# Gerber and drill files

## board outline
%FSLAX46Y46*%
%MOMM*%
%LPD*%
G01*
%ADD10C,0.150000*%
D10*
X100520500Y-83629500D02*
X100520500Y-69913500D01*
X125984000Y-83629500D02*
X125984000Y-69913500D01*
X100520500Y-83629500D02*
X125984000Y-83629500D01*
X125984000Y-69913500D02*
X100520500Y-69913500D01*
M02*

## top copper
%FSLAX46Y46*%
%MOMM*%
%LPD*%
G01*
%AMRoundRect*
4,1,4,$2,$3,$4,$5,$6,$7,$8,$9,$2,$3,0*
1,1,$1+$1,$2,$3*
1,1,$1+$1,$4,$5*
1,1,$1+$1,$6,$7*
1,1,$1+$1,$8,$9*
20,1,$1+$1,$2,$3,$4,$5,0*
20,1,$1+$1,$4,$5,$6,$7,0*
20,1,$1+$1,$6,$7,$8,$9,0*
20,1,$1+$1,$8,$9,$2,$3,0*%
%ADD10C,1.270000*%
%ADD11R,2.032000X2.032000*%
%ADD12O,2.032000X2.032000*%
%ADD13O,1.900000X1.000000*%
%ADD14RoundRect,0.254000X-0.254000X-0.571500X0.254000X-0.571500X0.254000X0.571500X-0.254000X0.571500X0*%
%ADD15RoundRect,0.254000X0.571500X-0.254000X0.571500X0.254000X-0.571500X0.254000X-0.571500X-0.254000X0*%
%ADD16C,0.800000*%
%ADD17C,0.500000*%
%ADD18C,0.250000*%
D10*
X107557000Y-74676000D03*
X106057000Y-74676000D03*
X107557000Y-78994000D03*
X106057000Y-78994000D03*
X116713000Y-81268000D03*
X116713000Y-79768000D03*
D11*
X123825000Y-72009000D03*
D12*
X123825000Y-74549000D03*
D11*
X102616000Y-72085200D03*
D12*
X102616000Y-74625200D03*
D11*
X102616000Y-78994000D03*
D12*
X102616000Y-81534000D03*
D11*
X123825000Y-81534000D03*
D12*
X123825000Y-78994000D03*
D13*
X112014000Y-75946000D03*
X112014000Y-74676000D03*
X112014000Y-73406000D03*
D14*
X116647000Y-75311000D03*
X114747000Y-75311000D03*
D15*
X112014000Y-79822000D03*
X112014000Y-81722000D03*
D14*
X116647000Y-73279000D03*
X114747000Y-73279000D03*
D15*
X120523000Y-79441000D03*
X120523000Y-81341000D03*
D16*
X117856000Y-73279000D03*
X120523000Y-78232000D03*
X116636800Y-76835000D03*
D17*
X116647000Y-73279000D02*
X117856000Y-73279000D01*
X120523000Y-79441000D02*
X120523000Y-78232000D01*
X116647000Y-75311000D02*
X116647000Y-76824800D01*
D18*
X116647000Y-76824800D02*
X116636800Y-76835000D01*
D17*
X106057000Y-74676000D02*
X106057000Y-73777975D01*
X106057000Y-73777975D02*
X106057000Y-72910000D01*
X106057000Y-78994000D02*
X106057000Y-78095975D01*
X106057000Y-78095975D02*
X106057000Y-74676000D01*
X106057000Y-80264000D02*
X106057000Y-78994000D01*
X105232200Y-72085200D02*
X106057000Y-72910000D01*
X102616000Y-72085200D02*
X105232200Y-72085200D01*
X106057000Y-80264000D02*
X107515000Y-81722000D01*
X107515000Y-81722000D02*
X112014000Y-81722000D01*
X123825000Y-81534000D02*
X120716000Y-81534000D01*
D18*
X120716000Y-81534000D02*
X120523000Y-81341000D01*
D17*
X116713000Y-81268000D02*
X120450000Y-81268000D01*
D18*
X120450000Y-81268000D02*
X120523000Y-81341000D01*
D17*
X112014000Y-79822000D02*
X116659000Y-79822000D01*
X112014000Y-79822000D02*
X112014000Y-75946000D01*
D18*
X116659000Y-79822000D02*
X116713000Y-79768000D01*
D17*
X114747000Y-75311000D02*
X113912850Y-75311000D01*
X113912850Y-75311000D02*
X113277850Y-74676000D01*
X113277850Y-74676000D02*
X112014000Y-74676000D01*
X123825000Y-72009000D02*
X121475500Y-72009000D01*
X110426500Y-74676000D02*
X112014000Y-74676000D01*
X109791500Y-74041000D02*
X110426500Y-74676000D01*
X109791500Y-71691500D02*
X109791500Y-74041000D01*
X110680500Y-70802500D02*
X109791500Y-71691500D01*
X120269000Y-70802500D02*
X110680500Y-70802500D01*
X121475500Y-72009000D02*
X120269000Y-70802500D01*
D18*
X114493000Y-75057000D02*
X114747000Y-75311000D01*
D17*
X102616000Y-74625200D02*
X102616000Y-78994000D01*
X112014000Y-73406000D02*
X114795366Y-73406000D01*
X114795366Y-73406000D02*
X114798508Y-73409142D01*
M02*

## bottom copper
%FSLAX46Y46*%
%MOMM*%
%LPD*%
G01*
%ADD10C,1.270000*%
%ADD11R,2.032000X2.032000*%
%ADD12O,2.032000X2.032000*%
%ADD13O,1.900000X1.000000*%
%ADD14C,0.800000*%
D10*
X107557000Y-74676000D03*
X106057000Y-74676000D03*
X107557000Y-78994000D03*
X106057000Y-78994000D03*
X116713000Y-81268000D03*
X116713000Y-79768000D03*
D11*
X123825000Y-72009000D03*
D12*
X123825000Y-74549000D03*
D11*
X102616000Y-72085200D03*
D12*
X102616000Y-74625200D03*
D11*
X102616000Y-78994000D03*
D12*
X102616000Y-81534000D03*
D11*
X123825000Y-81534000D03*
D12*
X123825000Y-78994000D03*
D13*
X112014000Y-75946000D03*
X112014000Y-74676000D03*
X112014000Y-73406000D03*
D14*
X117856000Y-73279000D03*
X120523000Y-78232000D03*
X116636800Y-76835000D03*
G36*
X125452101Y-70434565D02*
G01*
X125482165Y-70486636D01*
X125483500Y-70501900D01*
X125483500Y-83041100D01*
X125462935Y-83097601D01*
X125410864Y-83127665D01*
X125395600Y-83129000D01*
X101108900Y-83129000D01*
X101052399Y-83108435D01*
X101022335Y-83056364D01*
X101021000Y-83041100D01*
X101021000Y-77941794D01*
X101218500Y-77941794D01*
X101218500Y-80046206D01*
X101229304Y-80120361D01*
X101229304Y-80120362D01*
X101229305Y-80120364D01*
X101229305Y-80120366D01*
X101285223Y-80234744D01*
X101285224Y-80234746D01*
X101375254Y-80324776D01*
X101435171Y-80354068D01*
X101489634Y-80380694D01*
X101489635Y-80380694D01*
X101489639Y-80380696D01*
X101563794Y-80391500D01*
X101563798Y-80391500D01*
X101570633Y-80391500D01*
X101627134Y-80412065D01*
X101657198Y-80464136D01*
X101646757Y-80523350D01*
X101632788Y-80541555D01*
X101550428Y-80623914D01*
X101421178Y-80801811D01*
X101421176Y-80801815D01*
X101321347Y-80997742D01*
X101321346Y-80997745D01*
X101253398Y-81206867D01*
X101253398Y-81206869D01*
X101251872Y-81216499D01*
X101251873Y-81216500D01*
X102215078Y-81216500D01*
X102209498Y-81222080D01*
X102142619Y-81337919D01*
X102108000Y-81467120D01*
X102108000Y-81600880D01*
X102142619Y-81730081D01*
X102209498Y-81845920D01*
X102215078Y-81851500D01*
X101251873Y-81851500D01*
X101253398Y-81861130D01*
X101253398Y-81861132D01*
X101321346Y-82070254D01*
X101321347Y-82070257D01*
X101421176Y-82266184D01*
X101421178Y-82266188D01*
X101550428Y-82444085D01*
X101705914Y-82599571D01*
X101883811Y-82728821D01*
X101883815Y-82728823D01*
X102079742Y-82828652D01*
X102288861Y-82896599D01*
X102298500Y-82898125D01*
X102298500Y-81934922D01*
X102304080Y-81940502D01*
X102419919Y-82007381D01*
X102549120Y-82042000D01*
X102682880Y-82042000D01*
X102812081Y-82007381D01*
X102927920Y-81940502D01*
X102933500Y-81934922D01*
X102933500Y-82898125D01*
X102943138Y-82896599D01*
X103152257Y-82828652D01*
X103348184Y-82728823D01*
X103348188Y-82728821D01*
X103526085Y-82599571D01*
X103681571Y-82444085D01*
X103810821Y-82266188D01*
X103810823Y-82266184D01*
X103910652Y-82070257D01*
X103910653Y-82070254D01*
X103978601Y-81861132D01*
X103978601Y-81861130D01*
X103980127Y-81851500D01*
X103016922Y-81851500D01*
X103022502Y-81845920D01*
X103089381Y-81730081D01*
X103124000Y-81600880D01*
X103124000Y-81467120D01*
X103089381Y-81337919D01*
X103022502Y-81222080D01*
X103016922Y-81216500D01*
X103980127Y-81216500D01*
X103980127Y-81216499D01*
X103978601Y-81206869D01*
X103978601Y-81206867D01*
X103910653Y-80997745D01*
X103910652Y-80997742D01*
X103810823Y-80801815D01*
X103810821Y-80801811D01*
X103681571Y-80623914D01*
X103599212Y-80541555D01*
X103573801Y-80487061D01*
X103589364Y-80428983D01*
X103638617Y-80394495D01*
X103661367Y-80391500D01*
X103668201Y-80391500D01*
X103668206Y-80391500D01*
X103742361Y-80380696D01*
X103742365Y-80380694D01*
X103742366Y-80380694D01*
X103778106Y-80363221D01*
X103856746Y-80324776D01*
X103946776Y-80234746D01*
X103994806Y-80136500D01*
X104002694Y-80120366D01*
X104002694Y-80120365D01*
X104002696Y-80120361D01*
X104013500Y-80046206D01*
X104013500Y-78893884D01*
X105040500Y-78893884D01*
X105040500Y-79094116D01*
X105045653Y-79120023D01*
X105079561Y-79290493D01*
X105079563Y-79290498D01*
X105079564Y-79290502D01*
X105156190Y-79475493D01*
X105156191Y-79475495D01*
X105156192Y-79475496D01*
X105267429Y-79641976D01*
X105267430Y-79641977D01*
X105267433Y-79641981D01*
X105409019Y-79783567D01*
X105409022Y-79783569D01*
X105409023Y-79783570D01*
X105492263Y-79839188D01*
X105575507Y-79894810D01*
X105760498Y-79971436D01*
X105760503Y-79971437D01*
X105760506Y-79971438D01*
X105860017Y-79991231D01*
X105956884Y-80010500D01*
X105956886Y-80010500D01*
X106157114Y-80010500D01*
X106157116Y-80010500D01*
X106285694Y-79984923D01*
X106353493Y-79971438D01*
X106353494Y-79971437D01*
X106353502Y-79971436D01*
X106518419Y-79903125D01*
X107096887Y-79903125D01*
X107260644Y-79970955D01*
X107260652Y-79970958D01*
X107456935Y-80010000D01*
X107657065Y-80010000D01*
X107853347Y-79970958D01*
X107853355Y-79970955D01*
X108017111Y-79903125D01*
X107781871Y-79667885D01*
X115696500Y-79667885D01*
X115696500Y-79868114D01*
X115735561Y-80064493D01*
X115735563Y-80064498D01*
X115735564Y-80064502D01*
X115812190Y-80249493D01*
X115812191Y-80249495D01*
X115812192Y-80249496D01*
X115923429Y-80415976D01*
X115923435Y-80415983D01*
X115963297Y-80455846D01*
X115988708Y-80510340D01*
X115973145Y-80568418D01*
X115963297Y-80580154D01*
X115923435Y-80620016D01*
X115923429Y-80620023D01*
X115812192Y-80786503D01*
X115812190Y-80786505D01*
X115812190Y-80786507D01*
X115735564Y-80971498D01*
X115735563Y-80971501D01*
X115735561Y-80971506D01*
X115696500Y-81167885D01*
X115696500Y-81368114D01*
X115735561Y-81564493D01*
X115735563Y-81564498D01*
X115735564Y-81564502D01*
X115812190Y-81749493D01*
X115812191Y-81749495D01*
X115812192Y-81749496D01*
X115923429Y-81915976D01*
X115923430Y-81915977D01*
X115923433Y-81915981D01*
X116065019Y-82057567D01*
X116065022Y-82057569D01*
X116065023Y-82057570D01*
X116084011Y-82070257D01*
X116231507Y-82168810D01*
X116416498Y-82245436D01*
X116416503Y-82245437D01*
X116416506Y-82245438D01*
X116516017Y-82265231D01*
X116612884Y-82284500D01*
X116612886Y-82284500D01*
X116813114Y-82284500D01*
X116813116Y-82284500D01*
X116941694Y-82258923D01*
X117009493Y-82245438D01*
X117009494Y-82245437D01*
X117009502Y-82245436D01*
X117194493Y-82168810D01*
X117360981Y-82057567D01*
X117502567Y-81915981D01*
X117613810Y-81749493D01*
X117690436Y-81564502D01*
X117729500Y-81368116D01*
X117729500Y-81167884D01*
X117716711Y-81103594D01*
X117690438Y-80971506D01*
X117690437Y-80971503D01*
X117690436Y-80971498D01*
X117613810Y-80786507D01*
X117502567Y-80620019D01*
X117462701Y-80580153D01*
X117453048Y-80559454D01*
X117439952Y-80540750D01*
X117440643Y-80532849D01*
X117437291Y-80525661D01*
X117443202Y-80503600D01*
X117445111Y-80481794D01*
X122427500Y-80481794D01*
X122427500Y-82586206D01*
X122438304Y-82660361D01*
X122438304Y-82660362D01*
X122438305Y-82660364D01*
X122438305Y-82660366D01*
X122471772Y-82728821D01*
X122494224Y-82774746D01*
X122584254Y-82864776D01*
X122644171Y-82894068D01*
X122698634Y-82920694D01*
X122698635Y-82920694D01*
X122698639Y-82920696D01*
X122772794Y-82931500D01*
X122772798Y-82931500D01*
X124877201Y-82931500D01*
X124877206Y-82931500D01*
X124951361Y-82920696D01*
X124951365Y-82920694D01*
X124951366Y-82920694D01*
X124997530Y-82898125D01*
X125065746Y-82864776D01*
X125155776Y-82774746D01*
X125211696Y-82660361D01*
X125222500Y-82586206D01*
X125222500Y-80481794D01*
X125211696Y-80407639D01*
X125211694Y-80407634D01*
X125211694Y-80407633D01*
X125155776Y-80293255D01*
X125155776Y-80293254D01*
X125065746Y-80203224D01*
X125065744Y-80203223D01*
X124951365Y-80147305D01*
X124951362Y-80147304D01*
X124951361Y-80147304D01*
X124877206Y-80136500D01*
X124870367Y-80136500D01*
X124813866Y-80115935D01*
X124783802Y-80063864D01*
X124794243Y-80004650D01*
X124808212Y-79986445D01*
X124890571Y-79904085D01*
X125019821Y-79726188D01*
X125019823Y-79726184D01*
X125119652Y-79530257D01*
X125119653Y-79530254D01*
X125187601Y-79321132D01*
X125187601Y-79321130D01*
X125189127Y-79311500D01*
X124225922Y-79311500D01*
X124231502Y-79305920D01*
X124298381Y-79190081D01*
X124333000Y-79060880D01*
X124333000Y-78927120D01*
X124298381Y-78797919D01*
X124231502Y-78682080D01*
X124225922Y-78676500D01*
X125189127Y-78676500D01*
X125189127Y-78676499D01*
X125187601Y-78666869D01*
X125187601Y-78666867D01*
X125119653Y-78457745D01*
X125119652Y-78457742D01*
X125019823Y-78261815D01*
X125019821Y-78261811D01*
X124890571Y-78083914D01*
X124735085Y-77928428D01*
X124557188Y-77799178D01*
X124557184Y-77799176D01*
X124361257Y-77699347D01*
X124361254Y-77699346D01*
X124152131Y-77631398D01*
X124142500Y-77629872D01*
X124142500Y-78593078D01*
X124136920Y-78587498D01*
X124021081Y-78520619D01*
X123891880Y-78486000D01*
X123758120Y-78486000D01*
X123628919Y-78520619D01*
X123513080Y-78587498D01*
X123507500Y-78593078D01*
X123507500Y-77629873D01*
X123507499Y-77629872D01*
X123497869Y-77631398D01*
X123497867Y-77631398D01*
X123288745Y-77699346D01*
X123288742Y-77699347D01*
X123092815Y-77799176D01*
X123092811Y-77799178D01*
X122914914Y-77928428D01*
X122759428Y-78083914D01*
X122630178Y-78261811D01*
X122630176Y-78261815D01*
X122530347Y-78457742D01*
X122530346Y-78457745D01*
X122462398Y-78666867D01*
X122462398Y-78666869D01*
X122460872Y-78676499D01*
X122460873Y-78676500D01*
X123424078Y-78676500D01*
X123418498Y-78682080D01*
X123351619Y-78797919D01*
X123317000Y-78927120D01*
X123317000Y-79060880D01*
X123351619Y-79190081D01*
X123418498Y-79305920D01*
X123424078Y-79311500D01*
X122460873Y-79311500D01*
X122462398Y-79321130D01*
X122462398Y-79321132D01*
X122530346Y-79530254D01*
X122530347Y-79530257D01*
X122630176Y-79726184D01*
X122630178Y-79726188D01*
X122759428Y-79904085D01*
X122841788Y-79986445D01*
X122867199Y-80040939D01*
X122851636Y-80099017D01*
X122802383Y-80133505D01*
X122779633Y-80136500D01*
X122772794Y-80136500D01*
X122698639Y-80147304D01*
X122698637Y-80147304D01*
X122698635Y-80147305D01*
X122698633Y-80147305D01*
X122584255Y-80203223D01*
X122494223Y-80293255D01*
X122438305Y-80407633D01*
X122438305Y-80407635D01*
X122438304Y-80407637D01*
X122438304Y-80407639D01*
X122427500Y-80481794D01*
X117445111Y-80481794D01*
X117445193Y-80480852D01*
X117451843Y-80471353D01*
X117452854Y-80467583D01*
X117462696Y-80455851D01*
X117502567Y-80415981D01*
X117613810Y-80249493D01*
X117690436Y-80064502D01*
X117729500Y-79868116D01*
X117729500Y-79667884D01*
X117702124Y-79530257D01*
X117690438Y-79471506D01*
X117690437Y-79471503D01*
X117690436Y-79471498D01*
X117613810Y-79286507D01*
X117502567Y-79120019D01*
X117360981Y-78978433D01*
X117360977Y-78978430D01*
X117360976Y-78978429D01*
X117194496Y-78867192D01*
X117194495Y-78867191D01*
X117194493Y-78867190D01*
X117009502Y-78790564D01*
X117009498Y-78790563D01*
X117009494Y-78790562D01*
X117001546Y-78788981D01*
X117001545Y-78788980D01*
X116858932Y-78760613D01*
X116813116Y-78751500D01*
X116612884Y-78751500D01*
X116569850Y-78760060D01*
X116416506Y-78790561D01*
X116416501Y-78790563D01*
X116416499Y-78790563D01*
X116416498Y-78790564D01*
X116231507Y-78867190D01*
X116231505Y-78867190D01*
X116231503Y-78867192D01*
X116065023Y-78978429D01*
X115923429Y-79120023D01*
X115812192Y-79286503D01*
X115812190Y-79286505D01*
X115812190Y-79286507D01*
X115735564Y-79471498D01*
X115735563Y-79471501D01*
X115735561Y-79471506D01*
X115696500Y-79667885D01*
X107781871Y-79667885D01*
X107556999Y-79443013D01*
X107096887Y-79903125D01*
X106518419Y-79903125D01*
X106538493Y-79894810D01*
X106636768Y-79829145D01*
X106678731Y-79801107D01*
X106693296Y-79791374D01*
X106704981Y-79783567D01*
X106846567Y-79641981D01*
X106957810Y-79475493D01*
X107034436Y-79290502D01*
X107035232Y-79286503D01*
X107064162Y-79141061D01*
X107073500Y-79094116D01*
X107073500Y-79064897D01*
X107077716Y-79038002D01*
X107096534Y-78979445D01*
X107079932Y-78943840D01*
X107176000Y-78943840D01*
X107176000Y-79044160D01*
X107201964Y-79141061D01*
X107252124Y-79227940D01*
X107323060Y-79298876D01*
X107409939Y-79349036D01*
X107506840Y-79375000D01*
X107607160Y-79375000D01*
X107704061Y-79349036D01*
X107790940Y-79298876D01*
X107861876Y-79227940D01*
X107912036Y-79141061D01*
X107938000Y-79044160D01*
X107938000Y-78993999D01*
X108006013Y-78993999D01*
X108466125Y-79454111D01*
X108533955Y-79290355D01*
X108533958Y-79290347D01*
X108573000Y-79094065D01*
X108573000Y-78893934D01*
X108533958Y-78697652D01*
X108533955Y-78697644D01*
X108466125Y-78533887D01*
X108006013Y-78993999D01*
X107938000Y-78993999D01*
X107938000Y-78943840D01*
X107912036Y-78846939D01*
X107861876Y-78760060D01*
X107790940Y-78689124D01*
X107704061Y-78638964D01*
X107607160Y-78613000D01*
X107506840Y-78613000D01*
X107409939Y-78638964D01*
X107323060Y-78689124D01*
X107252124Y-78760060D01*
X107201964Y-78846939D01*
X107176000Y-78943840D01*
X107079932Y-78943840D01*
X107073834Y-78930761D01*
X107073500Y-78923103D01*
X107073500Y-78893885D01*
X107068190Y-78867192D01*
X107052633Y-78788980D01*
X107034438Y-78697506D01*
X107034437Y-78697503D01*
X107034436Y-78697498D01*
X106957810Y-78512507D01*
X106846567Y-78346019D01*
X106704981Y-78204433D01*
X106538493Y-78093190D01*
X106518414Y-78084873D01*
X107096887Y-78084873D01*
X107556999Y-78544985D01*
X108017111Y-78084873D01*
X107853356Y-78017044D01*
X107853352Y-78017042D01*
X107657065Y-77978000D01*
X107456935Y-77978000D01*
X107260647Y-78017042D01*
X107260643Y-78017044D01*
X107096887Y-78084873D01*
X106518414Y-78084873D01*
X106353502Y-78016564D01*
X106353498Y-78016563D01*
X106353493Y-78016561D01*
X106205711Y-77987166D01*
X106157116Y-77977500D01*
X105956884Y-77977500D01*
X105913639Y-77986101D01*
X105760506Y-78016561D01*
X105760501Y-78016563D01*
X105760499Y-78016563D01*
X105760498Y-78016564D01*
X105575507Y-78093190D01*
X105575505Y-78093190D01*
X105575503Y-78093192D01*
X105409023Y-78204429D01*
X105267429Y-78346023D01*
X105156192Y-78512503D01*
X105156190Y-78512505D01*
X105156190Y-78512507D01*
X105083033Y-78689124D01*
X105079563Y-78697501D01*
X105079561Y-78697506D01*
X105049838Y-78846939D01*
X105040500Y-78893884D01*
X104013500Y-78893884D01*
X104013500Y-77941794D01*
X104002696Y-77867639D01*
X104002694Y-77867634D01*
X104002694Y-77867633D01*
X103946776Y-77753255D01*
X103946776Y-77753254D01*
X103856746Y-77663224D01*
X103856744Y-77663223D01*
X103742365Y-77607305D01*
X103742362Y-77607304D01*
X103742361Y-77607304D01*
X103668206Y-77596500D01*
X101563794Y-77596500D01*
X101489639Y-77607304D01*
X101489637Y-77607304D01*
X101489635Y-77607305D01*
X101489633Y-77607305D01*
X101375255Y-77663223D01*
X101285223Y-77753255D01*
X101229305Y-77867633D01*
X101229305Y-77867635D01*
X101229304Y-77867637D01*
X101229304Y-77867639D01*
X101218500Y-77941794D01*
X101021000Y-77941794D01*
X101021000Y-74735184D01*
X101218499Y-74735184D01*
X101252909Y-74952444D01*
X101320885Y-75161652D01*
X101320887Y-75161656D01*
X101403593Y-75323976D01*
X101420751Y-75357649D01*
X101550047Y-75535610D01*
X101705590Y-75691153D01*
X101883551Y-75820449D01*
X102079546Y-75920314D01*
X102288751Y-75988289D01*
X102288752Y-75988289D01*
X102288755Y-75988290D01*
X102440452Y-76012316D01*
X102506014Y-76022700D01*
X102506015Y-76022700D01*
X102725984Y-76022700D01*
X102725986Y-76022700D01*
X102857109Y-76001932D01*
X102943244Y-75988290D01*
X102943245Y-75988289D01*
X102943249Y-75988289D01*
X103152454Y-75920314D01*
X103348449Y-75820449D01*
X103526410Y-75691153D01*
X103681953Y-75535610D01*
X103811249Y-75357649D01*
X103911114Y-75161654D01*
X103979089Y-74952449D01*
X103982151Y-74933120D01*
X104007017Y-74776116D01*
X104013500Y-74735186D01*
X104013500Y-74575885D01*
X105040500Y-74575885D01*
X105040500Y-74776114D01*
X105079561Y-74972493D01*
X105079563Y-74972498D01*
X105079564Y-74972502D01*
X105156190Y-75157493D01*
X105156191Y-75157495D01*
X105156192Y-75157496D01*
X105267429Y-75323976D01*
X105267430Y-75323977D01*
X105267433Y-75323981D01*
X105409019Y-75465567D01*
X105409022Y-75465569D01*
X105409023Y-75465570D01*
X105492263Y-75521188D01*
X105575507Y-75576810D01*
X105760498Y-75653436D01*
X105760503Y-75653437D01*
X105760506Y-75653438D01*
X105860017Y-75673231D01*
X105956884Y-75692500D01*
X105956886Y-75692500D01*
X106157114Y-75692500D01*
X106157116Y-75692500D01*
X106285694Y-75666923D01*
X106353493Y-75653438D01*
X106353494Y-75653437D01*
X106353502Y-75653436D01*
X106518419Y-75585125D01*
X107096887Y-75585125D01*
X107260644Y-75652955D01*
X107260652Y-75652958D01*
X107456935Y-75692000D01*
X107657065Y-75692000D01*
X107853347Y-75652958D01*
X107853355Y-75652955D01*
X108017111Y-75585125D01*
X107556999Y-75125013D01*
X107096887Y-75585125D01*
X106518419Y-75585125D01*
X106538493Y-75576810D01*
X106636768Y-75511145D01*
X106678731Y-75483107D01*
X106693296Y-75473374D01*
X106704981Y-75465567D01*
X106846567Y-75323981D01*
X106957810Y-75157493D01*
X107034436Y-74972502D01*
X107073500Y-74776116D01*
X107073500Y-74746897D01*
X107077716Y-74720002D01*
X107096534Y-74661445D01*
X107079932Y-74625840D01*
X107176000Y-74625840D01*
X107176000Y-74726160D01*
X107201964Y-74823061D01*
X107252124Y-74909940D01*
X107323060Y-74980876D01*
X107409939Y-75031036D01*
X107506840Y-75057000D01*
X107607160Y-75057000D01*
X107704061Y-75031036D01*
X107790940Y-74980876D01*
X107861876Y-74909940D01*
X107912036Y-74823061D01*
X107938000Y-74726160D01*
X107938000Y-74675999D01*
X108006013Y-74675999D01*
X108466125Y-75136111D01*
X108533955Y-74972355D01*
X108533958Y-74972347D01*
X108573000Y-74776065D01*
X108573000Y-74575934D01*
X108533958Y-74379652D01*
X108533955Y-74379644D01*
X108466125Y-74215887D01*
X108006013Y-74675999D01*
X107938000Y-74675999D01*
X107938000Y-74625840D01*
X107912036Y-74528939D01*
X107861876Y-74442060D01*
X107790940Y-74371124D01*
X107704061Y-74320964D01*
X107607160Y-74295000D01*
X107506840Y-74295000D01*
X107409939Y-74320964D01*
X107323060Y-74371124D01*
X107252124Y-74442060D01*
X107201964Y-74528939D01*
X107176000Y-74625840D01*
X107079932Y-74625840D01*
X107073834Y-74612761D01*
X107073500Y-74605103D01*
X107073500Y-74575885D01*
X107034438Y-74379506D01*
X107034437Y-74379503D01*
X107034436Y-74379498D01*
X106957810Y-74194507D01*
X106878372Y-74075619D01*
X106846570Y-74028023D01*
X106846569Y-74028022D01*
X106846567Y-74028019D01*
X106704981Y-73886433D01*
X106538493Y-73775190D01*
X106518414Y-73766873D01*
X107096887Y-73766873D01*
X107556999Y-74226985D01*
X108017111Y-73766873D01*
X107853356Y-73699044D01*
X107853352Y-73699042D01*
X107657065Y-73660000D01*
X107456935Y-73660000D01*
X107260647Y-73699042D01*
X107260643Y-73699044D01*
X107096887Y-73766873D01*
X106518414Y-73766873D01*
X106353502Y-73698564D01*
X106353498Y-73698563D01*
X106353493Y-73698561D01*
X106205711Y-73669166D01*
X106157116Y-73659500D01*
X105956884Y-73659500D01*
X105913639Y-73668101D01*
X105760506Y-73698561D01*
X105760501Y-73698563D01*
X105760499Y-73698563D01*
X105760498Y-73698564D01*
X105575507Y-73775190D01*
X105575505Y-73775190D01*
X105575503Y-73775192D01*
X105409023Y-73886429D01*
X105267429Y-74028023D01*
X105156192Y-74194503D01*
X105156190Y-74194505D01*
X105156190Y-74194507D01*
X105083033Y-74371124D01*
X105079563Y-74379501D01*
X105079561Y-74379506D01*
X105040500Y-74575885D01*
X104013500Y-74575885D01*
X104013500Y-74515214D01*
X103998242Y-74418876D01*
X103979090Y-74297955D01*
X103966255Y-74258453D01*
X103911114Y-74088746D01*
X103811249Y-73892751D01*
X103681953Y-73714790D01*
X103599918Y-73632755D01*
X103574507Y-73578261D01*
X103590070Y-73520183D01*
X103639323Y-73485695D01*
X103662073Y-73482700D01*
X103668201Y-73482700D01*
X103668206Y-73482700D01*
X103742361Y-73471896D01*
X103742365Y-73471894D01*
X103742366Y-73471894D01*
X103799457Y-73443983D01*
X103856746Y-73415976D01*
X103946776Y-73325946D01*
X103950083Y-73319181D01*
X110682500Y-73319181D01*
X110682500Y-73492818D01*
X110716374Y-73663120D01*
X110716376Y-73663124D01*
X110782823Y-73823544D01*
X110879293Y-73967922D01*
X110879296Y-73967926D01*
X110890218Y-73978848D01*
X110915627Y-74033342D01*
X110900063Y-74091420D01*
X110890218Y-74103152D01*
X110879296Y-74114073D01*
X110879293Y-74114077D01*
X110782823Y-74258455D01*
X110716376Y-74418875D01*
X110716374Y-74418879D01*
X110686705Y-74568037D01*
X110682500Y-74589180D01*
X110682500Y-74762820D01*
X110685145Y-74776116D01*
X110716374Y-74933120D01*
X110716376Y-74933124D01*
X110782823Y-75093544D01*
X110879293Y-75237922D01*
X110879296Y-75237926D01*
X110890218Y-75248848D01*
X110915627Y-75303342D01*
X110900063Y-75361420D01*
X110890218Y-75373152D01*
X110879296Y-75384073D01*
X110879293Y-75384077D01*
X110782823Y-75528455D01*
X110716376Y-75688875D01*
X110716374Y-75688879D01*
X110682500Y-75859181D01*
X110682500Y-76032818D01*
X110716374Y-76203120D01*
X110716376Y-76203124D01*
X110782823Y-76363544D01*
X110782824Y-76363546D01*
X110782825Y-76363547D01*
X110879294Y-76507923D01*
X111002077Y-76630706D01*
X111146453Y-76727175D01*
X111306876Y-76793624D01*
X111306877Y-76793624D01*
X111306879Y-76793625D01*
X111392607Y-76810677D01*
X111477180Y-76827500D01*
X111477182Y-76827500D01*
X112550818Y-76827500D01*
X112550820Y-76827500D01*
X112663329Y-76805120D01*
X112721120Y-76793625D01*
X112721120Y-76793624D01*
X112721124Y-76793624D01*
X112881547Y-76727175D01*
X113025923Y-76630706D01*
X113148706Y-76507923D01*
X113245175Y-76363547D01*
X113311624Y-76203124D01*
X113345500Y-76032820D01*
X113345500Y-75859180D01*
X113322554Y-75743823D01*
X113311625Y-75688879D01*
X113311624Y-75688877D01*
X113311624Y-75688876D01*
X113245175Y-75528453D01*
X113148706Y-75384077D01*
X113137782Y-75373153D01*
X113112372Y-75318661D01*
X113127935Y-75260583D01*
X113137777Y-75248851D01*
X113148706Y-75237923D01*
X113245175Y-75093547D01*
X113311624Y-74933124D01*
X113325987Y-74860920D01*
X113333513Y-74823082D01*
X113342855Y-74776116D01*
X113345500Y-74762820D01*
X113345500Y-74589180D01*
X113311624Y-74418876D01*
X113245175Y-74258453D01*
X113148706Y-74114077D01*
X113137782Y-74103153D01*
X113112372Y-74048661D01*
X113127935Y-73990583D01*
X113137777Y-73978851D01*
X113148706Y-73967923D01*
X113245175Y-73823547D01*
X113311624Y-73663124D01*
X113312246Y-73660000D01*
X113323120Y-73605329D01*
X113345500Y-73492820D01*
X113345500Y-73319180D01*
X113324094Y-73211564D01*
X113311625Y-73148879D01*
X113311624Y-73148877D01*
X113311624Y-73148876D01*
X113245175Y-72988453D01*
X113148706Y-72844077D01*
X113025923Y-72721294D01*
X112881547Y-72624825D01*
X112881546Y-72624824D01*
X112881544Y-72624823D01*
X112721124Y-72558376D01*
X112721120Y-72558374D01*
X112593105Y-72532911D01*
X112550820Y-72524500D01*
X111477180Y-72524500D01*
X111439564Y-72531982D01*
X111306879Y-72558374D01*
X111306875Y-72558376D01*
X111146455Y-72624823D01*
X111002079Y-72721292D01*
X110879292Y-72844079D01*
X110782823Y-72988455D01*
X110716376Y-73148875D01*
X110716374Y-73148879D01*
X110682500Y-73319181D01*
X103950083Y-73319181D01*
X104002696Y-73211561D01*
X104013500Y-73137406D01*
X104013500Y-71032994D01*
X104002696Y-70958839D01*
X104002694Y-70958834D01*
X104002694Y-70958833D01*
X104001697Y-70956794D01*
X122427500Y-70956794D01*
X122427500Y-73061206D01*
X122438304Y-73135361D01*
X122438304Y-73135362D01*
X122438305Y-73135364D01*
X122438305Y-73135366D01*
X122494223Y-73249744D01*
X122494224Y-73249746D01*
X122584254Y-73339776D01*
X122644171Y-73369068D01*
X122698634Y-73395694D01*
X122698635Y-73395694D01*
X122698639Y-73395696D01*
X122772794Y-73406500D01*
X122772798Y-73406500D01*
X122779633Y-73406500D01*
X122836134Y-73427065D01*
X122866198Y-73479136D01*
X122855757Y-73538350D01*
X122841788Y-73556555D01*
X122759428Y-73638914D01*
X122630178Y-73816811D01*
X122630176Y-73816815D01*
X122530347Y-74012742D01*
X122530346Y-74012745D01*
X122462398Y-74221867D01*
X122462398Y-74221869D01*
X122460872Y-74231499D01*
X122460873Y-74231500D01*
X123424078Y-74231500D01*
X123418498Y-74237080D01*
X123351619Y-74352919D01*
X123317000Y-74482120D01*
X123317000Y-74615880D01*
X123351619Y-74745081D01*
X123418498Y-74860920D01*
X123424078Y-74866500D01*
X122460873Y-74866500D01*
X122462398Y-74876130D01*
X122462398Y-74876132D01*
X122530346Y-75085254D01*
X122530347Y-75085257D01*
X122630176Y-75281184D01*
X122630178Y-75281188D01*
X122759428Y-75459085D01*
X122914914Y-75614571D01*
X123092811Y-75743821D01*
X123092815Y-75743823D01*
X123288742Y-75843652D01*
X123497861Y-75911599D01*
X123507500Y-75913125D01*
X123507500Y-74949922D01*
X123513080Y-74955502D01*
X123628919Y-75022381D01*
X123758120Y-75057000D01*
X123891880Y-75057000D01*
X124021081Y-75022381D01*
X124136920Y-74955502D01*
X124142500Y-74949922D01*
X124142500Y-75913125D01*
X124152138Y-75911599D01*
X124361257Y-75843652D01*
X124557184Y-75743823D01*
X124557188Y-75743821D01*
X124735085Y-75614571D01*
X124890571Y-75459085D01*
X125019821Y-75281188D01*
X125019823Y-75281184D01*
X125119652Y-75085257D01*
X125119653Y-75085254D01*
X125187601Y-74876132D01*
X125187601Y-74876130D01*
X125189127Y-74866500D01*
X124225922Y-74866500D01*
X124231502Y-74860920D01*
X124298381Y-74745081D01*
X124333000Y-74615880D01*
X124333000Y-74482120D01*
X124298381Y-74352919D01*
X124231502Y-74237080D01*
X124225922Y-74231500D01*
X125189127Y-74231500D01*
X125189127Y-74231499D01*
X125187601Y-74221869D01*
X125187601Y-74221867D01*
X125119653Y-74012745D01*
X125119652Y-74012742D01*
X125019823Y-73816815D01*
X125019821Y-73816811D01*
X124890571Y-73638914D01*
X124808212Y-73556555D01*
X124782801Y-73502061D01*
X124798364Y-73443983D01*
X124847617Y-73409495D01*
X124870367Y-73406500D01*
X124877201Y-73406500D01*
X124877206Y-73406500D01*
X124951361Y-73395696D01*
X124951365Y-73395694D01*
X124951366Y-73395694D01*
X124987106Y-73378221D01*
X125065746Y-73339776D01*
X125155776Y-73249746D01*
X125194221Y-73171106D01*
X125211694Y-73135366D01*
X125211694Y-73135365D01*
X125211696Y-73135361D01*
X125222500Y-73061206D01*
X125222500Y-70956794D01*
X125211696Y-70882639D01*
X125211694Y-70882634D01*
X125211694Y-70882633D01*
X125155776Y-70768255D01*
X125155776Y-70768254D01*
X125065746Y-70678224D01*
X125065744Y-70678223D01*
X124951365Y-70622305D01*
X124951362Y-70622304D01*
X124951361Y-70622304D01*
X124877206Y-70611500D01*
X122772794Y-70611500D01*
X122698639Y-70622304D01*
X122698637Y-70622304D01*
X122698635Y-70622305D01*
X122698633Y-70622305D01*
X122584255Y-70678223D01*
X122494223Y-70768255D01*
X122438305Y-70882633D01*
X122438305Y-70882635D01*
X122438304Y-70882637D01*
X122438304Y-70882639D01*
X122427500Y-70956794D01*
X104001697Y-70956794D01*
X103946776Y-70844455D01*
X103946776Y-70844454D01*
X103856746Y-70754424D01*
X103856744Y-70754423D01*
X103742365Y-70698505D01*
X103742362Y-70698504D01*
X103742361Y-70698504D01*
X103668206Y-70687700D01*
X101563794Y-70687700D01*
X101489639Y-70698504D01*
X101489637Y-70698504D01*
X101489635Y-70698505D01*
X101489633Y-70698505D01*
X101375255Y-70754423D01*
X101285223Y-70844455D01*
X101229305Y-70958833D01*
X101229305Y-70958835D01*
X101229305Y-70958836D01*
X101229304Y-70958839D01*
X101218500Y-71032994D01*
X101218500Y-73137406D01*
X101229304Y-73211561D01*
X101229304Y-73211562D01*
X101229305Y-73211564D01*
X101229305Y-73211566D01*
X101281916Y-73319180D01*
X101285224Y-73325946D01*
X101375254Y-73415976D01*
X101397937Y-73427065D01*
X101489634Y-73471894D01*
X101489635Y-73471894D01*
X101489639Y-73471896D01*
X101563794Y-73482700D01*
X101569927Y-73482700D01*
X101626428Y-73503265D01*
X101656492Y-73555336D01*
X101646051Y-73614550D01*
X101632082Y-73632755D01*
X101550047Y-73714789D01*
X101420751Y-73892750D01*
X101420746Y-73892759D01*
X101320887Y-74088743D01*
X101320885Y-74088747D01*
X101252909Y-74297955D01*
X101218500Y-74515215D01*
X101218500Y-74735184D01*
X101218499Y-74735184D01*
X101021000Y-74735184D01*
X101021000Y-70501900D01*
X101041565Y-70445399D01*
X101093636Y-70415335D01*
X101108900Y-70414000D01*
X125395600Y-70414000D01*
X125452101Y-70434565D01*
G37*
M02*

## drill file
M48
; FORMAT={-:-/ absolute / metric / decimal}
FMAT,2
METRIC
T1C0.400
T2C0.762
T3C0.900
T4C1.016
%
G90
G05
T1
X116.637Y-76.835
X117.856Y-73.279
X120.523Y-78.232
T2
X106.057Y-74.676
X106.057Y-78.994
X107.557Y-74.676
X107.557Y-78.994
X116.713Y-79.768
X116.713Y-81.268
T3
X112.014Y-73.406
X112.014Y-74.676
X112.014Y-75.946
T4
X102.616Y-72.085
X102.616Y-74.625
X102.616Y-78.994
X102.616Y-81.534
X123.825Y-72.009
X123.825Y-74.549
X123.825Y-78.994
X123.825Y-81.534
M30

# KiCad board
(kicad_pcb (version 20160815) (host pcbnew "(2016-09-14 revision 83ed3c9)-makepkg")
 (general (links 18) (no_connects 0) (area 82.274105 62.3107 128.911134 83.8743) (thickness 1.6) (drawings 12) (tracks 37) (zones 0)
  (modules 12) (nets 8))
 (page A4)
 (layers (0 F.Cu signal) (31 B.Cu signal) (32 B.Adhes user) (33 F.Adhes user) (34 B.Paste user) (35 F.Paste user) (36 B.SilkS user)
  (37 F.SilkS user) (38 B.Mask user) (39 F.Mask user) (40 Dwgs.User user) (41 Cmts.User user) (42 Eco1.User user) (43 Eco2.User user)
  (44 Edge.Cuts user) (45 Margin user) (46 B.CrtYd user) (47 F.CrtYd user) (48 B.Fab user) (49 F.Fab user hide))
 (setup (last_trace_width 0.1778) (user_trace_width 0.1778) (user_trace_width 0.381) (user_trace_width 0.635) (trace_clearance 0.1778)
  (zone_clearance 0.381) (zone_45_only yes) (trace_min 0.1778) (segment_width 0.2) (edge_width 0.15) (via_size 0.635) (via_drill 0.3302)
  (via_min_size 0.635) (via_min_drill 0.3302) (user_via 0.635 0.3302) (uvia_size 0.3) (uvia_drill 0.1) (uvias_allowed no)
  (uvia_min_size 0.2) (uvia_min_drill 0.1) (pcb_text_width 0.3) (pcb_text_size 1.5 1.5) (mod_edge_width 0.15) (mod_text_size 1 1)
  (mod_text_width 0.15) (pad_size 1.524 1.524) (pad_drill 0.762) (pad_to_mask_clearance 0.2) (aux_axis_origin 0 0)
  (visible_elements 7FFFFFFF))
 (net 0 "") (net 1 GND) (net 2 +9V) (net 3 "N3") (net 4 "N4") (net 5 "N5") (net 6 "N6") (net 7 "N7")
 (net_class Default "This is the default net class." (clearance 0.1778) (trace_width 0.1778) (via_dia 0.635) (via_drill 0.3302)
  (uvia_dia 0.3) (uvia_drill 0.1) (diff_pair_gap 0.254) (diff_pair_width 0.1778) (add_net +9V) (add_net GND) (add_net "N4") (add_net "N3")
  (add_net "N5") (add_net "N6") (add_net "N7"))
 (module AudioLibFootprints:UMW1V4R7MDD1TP (layer F.Cu) (at 106.807 74.676)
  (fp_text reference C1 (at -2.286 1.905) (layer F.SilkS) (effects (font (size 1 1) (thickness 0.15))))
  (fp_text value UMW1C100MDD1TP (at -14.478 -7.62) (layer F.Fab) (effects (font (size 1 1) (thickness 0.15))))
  (pad 2 thru_hole circle (at 0.75 0) (size 1.27 1.27) (drill 0.762) (layers *.Cu *.Mask) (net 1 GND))
  (pad 1 thru_hole circle (at -0.75 0) (size 1.27 1.27) (drill 0.762) (layers *.Cu *.Mask) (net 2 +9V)))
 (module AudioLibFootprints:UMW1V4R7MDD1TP (layer F.Cu) (at 106.807 78.994)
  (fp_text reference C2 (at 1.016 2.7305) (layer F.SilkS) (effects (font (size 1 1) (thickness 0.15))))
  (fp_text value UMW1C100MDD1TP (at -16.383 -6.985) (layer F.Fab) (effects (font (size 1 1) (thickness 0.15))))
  (pad 2 thru_hole circle (at 0.75 0) (size 1.27 1.27) (drill 0.762) (layers *.Cu *.Mask) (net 1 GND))
  (pad 1 thru_hole circle (at -0.75 0) (size 1.27 1.27) (drill 0.762) (layers *.Cu *.Mask) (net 2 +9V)))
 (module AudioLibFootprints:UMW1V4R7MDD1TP (layer F.Cu) (at 116.713 80.518 270)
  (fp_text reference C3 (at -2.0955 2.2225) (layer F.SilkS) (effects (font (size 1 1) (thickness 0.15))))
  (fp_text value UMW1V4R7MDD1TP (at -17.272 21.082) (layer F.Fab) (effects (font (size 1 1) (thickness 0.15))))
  (pad 2 thru_hole circle (at 0.75 0 270) (size 1.27 1.27) (drill 0.762) (layers *.Cu *.Mask) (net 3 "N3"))
  (pad 1 thru_hole circle (at -0.75 0 270) (size 1.27 1.27) (drill 0.762) (layers *.Cu *.Mask) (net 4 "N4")))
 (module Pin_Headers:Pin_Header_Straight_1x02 (layer F.Cu) (at 123.825 72.009)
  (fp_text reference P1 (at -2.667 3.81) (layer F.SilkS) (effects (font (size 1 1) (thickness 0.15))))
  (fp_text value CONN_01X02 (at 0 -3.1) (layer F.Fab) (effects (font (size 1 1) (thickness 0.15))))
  (pad 1 thru_hole rect (at 0 0) (size 2.032 2.032) (drill 1.016) (layers *.Cu *.Mask F.SilkS) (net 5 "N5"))
  (pad 2 thru_hole oval (at 0 2.54) (size 2.032 2.032) (drill 1.016) (layers *.Cu *.Mask F.SilkS) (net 1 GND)))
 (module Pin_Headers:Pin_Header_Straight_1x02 (layer F.Cu) (at 102.616 72.0852)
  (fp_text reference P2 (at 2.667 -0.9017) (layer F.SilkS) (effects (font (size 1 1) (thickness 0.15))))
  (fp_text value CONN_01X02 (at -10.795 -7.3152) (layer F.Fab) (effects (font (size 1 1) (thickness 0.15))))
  (pad 1 thru_hole rect (at 0 0) (size 2.032 2.032) (drill 1.016) (layers *.Cu *.Mask F.SilkS) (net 2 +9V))
  (pad 2 thru_hole oval (at 0 2.54) (size 2.032 2.032) (drill 1.016) (layers *.Cu *.Mask F.SilkS) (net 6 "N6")))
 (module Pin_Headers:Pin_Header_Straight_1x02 (layer F.Cu) (at 102.616 78.994)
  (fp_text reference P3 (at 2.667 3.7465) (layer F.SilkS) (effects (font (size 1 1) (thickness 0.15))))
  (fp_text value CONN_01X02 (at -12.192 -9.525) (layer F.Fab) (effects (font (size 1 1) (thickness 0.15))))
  (pad 1 thru_hole rect (at 0 0) (size 2.032 2.032) (drill 1.016) (layers *.Cu *.Mask F.SilkS) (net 6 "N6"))
  (pad 2 thru_hole oval (at 0 2.54) (size 2.032 2.032) (drill 1.016) (layers *.Cu *.Mask F.SilkS) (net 1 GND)))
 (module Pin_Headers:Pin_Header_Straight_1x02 (layer F.Cu) (at 123.825 81.534 180)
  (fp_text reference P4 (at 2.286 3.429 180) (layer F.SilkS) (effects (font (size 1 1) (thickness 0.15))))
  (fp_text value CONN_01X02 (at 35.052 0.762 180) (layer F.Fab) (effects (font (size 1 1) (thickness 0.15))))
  (pad 1 thru_hole rect (at 0 0 180) (size 2.032 2.032) (drill 1.016) (layers *.Cu *.Mask F.SilkS) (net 3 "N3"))
  (pad 2 thru_hole oval (at 0 2.54 180) (size 2.032 2.032) (drill 1.016) (layers *.Cu *.Mask F.SilkS) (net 1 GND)))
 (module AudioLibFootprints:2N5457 (layer F.Cu) (at 112.014 74.676)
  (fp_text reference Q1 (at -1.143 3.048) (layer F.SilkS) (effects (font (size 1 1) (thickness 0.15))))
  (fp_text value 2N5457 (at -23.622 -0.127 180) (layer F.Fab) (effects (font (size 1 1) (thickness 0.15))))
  (pad 1 thru_hole oval (at 0 1.27) (size 1.9 1) (drill 0.9) (layers *.Cu *.Mask) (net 4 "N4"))
  (pad 2 thru_hole oval (at 0 0) (size 1.9 1) (drill 0.9) (layers *.Cu *.Mask) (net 5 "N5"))
  (pad 3 thru_hole oval (at 0 -1.27) (size 1.9 1) (drill 0.9) (layers *.Cu *.Mask) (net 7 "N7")))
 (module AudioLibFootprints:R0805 (layer F.Cu) (at 115.697 75.311)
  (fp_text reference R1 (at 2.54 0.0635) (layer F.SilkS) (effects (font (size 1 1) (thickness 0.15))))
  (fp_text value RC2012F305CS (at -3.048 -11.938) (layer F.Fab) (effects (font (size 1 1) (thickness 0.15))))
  (pad 2 smd roundrect (at 0.95 0) (size 1.016 1.651) (layers F.Cu F.Paste F.Mask) (roundrect_rratio 0.25) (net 1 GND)
   (solder_mask_margin 0.102))
  (pad 1 smd roundrect (at -0.95 0) (size 1.016 1.651) (layers F.Cu F.Paste F.Mask) (roundrect_rratio 0.25) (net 5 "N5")
   (solder_mask_margin 0.102)))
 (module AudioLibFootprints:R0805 (layer F.Cu) (at 112.014 80.772 90)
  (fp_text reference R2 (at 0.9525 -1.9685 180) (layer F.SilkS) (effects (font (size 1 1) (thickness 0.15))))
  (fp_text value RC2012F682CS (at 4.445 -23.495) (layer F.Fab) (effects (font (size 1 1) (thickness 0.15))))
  (pad 2 smd roundrect (at 0.95 0 90) (size 1.016 1.651) (layers F.Cu F.Paste F.Mask) (roundrect_rratio 0.25) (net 4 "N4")
   (solder_mask_margin 0.102))
  (pad 1 smd roundrect (at -0.95 0 90) (size 1.016 1.651) (layers F.Cu F.Paste F.Mask) (roundrect_rratio 0.25) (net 2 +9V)
   (solder_mask_margin 0.102)))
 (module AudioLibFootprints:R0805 (layer F.Cu) (at 115.697 73.279)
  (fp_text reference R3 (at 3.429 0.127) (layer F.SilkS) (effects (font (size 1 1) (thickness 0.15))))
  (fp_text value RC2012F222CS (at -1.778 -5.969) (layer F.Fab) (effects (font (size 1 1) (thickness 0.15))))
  (pad 2 smd roundrect (at 0.95 0) (size 1.016 1.651) (layers F.Cu F.Paste F.Mask) (roundrect_rratio 0.25) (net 1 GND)
   (solder_mask_margin 0.102))
  (pad 1 smd roundrect (at -0.95 0) (size 1.016 1.651) (layers F.Cu F.Paste F.Mask) (roundrect_rratio 0.25) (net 7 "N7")
   (solder_mask_margin 0.102)))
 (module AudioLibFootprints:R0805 (layer F.Cu) (at 120.523 80.391 90)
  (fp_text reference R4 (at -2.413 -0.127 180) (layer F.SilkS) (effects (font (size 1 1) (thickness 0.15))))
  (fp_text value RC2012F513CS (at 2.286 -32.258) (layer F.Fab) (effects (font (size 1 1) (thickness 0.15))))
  (pad 2 smd roundrect (at 0.95 0 90) (size 1.016 1.651) (layers F.Cu F.Paste F.Mask) (roundrect_rratio 0.25) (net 1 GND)
   (solder_mask_margin 0.102))
  (pad 1 smd roundrect (at -0.95 0 90) (size 1.016 1.651) (layers F.Cu F.Paste F.Mask) (roundrect_rratio 0.25) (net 3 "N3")
   (solder_mask_margin 0.102)))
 (gr_line (start 100.5205 83.6295) (end 100.5205 69.9135) (angle 90) (layer Edge.Cuts) (width 0.15))
 (gr_line (start 125.984 83.6295) (end 125.984 69.9135) (angle 90) (layer Edge.Cuts) (width 0.15))
 (gr_line (start 100.5205 83.6295) (end 125.984 83.6295) (angle 90) (layer Edge.Cuts) (width 0.15))
 (gr_line (start 125.984 69.9135) (end 100.5205 69.9135) (angle 90) (layer Edge.Cuts) (width 0.15))
 (segment (start 116.647 73.279) (end 117.856 73.279) (width 0.5) (layer F.Cu) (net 1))
 (via (at 117.856 73.279) (size 0.8) (drill 0.4) (layers F.Cu B.Cu) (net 1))
 (segment (start 120.523 79.441) (end 120.523 78.232) (width 0.5) (layer F.Cu) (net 1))
 (via (at 120.523 78.232) (size 0.8) (drill 0.4) (layers F.Cu B.Cu) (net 1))
 (segment (start 116.647 75.311) (end 116.647 76.8248) (width 0.5) (layer F.Cu) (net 1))
 (segment (start 116.647 76.8248) (end 116.6368 76.835) (width 0.25) (layer F.Cu) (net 1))
 (via (at 116.6368 76.835) (size 0.8) (drill 0.4) (layers F.Cu B.Cu) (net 1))
 (segment (start 106.057 74.676) (end 106.057 73.777975) (width 0.5) (layer F.Cu) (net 2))
 (segment (start 106.057 73.777975) (end 106.057 72.91) (width 0.5) (layer F.Cu) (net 2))
 (segment (start 106.057 78.994) (end 106.057 78.095975) (width 0.5) (layer F.Cu) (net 2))
 (segment (start 106.057 78.095975) (end 106.057 74.676) (width 0.5) (layer F.Cu) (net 2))
 (segment (start 106.057 80.264) (end 106.057 78.994) (width 0.5) (layer F.Cu) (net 2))
 (segment (start 105.2322 72.0852) (end 106.057 72.91) (width 0.5) (layer F.Cu) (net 2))
 (segment (start 102.616 72.0852) (end 105.2322 72.0852) (width 0.5) (layer F.Cu) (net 2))
 (segment (start 106.057 80.264) (end 107.515 81.722) (width 0.5) (layer F.Cu) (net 2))
 (segment (start 107.515 81.722) (end 112.014 81.722) (width 0.5) (layer F.Cu) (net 2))
 (segment (start 123.825 81.534) (end 120.716 81.534) (width 0.5) (layer F.Cu) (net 3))
 (segment (start 120.716 81.534) (end 120.523 81.341) (width 0.25) (layer F.Cu) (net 3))
 (segment (start 116.713 81.268) (end 120.45 81.268) (width 0.5) (layer F.Cu) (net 3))
 (segment (start 120.45 81.268) (end 120.523 81.341) (width 0.25) (layer F.Cu) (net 3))
 (segment (start 112.014 79.822) (end 116.659 79.822) (width 0.5) (layer F.Cu) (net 4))
 (segment (start 112.014 79.822) (end 112.014 75.946) (width 0.5) (layer F.Cu) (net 4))
 (segment (start 116.659 79.822) (end 116.713 79.768) (width 0.25) (layer F.Cu) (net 4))
 (segment (start 114.747 75.311) (end 113.91285 75.311) (width 0.5) (layer F.Cu) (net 5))
 (segment (start 113.91285 75.311) (end 113.27785 74.676) (width 0.5) (layer F.Cu) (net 5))
 (segment (start 113.27785 74.676) (end 112.014 74.676) (width 0.5) (layer F.Cu) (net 5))
 (segment (start 123.825 72.009) (end 121.4755 72.009) (width 0.5) (layer F.Cu) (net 5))
 (segment (start 110.4265 74.676) (end 112.014 74.676) (width 0.5) (layer F.Cu) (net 5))
 (segment (start 109.7915 74.041) (end 110.4265 74.676) (width 0.5) (layer F.Cu) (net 5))
 (segment (start 109.7915 71.6915) (end 109.7915 74.041) (width 0.5) (layer F.Cu) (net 5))
 (segment (start 110.6805 70.8025) (end 109.7915 71.6915) (width 0.5) (layer F.Cu) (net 5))
 (segment (start 120.269 70.8025) (end 110.6805 70.8025) (width 0.5) (layer F.Cu) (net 5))
 (segment (start 121.4755 72.009) (end 120.269 70.8025) (width 0.5) (layer F.Cu) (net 5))
 (segment (start 114.493 75.057) (end 114.747 75.311) (width 0.25) (layer F.Cu) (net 5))
 (segment (start 102.616 74.6252) (end 102.616 78.994) (width 0.5) (layer F.Cu) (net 6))
 (segment (start 112.014 73.406) (end 114.795366 73.406) (width 0.5) (layer F.Cu) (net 7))
 (segment (start 114.795366 73.406) (end 114.798508 73.409142) (width 0.5) (layer F.Cu) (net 7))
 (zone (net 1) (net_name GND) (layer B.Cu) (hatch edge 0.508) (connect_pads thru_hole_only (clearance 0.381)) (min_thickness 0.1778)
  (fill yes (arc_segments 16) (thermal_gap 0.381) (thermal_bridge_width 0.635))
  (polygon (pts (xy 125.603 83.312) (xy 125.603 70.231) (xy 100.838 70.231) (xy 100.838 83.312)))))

